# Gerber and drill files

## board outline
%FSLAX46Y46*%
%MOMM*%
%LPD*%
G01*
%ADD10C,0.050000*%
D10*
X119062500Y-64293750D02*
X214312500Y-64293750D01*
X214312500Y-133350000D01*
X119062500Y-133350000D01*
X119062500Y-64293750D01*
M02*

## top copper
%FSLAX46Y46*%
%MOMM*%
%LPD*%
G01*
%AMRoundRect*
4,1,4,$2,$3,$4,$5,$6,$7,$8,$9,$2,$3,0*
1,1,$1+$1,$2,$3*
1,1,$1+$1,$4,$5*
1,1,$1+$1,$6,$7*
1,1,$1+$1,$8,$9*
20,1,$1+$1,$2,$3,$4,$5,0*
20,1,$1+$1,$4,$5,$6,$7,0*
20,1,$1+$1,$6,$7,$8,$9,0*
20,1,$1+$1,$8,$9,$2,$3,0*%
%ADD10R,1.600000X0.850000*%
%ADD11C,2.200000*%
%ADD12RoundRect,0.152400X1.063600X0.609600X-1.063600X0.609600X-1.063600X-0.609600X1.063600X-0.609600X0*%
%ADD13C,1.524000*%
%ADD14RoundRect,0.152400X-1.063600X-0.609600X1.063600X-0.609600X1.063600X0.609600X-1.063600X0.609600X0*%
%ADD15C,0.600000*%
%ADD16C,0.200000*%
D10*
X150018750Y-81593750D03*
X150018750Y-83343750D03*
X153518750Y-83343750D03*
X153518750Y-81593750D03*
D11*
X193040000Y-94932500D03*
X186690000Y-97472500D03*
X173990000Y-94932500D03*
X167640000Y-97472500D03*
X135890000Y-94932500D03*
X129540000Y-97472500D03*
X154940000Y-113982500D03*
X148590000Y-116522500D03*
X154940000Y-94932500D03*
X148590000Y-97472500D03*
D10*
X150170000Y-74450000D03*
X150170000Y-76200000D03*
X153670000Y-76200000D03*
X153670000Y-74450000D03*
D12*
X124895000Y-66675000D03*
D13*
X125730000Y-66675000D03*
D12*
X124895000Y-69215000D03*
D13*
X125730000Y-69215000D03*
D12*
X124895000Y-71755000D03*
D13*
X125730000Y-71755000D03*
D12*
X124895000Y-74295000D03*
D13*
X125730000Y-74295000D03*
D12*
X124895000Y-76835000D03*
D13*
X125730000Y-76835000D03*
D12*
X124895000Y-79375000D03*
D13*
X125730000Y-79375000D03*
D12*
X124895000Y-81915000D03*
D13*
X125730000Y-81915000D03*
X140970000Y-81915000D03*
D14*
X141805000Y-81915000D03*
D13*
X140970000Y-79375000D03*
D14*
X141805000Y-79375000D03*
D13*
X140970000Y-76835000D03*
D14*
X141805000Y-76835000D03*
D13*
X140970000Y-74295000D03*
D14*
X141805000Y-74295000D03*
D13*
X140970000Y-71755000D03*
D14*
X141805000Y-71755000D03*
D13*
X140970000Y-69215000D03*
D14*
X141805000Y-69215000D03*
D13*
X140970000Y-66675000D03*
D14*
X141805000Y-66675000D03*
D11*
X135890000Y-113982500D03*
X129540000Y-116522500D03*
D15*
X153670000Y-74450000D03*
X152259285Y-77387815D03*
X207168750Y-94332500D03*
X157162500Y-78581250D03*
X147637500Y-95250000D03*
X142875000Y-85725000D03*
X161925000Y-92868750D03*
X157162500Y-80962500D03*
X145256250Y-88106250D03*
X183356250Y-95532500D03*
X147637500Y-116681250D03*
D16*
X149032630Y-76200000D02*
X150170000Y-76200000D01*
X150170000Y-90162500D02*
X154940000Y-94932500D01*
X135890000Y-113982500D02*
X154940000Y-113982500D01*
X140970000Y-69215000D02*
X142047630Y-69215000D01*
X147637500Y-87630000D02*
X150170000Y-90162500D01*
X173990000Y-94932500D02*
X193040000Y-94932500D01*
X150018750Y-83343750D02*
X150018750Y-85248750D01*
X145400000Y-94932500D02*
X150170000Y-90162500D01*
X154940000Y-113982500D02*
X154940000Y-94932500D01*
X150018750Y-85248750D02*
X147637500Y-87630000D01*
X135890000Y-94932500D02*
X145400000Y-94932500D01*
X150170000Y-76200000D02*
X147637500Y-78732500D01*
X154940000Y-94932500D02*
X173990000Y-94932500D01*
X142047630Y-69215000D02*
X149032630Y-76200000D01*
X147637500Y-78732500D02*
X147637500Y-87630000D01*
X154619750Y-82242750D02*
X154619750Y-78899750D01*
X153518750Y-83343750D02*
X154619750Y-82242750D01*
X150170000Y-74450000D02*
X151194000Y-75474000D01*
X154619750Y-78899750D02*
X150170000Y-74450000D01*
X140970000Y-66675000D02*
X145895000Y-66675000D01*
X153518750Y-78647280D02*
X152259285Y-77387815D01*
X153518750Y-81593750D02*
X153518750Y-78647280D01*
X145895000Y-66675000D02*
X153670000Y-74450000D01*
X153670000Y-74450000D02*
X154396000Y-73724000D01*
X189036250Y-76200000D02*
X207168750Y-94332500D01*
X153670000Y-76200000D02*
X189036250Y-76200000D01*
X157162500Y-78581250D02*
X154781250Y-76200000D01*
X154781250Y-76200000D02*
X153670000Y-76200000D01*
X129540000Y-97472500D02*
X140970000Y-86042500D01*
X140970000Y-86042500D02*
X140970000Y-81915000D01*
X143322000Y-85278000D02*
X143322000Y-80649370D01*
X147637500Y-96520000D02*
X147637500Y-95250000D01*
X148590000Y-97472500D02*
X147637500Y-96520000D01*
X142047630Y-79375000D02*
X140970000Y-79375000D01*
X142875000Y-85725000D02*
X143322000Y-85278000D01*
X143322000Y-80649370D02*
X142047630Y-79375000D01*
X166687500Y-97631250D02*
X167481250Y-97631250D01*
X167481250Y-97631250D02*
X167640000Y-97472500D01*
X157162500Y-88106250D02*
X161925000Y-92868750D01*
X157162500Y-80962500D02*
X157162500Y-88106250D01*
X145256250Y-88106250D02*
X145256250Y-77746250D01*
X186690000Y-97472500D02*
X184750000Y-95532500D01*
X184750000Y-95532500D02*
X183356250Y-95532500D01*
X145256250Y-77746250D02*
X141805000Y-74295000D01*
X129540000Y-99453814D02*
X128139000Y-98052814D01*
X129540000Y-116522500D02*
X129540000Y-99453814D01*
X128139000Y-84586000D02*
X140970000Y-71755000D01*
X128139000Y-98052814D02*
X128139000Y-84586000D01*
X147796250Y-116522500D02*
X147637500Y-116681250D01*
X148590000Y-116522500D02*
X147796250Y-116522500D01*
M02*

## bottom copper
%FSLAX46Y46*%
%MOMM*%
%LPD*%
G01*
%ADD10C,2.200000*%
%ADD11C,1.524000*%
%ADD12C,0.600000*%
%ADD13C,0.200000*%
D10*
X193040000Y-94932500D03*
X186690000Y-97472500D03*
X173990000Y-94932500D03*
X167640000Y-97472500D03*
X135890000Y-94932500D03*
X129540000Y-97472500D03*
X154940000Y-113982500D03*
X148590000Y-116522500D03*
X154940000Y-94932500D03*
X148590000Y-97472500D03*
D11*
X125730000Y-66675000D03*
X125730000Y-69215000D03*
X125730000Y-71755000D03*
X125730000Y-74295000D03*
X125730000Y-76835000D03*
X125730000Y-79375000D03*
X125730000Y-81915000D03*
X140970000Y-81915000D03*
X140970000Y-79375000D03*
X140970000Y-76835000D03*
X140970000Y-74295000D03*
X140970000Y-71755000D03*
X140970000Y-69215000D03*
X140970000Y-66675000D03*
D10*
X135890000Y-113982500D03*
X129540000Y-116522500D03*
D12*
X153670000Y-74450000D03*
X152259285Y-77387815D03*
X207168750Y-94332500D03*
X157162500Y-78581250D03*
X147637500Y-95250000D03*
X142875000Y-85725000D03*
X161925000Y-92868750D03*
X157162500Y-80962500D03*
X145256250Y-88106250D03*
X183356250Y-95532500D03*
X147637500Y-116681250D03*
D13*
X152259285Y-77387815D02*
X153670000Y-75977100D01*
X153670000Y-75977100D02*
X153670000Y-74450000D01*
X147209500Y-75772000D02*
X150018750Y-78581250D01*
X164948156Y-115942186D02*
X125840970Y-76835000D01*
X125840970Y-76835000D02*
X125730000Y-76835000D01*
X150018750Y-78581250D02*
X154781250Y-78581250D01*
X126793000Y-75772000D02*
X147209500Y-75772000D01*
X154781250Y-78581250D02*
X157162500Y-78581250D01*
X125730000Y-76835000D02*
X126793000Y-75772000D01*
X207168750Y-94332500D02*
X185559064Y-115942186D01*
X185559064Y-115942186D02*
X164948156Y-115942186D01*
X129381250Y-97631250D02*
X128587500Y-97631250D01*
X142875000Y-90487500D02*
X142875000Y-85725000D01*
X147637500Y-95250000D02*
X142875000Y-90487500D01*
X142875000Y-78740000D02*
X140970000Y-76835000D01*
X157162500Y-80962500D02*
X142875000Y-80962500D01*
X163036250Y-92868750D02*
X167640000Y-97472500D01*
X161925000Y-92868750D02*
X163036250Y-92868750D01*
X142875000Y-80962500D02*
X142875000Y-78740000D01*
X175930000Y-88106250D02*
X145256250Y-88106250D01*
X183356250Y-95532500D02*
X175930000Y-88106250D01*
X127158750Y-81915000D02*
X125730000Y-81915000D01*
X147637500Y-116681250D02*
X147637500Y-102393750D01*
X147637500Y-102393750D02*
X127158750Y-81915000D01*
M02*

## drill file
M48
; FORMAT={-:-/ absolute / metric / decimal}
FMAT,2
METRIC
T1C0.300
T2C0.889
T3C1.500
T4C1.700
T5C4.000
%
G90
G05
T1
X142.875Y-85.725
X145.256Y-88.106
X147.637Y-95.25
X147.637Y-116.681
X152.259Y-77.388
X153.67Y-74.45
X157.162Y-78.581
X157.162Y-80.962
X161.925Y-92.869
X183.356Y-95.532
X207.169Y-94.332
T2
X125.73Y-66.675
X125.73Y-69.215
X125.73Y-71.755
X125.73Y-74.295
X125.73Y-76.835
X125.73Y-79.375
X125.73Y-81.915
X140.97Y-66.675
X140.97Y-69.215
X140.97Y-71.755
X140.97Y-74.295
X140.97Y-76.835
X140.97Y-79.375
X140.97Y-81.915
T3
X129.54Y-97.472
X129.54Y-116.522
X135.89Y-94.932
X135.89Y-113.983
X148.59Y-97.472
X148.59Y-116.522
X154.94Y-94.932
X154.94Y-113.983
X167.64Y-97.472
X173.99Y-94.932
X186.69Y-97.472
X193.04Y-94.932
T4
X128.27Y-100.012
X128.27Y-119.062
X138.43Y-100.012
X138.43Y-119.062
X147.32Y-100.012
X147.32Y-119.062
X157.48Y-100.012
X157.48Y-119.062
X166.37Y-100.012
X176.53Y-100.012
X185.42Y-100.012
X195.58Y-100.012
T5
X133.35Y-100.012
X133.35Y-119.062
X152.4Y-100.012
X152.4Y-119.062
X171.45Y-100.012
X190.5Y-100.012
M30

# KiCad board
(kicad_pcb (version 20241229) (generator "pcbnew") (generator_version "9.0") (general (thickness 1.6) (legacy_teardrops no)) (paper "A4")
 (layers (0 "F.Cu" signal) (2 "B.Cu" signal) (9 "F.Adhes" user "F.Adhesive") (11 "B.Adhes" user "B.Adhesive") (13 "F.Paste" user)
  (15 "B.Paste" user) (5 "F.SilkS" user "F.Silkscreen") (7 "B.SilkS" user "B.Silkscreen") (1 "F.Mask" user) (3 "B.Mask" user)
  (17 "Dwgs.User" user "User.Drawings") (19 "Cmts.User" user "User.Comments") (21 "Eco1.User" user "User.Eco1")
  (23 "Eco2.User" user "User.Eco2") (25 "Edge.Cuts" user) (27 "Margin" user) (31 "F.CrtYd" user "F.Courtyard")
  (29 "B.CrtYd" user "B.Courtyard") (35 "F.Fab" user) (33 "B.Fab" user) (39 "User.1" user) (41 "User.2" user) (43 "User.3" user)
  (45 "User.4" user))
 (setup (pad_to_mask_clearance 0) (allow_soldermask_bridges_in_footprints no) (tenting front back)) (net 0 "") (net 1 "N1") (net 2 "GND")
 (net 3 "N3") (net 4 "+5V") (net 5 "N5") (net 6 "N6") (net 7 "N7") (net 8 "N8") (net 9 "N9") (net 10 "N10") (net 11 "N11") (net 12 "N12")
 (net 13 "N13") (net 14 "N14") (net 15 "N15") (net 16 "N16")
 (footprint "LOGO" (layer "F.Cu") (at 169.754101 70.000013)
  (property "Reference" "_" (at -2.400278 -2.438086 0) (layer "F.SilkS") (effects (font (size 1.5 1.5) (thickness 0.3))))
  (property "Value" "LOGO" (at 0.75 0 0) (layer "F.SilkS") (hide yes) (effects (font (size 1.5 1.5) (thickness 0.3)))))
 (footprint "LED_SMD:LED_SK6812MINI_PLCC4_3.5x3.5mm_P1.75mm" (layer "F.Cu") (at 151.76875 82.46875)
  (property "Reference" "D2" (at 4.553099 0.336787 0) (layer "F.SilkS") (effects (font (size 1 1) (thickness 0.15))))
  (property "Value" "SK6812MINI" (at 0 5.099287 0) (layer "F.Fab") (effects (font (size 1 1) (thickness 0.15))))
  (pad "1" smd rect (at -1.75 -0.875) (size 1.6 0.85) (layers "F.Cu" "F.Mask" "F.Paste") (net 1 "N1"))
  (pad "2" smd rect (at -1.75 0.875) (size 1.6 0.85) (layers "F.Cu" "F.Mask" "F.Paste") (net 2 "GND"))
  (pad "3" smd rect (at 1.75 0.875) (size 1.6 0.85) (layers "F.Cu" "F.Mask" "F.Paste") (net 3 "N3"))
  (pad "4" smd rect (at 1.75 -0.875) (size 1.6 0.85) (layers "F.Cu" "F.Mask" "F.Paste") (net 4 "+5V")))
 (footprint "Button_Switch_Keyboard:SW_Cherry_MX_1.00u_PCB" (layer "F.Cu") (at 193.04 94.9325)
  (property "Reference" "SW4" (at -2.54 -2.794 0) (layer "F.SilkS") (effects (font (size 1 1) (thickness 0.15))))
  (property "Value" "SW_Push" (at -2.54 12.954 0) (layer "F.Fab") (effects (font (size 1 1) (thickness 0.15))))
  (pad "" np_thru_hole circle (at -7.62 5.08) (size 1.7 1.7) (drill 1.7) (layers "*.Cu" "*.Mask"))
  (pad "" np_thru_hole circle (at -2.54 5.08) (size 4 4) (drill 4) (layers "*.Cu" "*.Mask"))
  (pad "" np_thru_hole circle (at 2.54 5.08) (size 1.7 1.7) (drill 1.7) (layers "*.Cu" "*.Mask"))
  (pad "1" thru_hole circle (at 0 0) (size 2.2 2.2) (drill 1.5) (layers "*.Cu" "*.Mask") (remove_unused_layers no) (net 2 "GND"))
  (pad "2" thru_hole circle (at -6.35 2.54) (size 2.2 2.2) (drill 1.5) (layers "*.Cu" "*.Mask") (remove_unused_layers no) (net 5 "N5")))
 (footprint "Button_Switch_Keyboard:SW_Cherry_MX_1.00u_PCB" (layer "F.Cu") (at 173.99 94.9325)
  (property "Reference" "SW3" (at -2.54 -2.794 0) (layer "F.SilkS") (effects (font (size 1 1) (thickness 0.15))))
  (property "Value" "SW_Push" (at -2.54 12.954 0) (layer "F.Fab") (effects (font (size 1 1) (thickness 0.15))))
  (pad "" np_thru_hole circle (at -7.62 5.08) (size 1.7 1.7) (drill 1.7) (layers "*.Cu" "*.Mask"))
  (pad "" np_thru_hole circle (at -2.54 5.08) (size 4 4) (drill 4) (layers "*.Cu" "*.Mask"))
  (pad "" np_thru_hole circle (at 2.54 5.08) (size 1.7 1.7) (drill 1.7) (layers "*.Cu" "*.Mask"))
  (pad "1" thru_hole circle (at 0 0) (size 2.2 2.2) (drill 1.5) (layers "*.Cu" "*.Mask") (remove_unused_layers no) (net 2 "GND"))
  (pad "2" thru_hole circle (at -6.35 2.54) (size 2.2 2.2) (drill 1.5) (layers "*.Cu" "*.Mask") (remove_unused_layers no) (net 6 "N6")))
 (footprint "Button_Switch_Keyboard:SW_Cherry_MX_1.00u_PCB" (layer "F.Cu") (at 135.89 94.9325)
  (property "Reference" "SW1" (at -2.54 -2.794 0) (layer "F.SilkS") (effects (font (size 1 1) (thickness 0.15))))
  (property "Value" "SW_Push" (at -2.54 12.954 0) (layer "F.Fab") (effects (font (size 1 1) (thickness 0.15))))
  (pad "" np_thru_hole circle (at -7.62 5.08) (size 1.7 1.7) (drill 1.7) (layers "*.Cu" "*.Mask"))
  (pad "" np_thru_hole circle (at -2.54 5.08) (size 4 4) (drill 4) (layers "*.Cu" "*.Mask"))
  (pad "" np_thru_hole circle (at 2.54 5.08) (size 1.7 1.7) (drill 1.7) (layers "*.Cu" "*.Mask"))
  (pad "1" thru_hole circle (at 0 0) (size 2.2 2.2) (drill 1.5) (layers "*.Cu" "*.Mask") (remove_unused_layers no) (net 2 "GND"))
  (pad "2" thru_hole circle (at -6.35 2.54) (size 2.2 2.2) (drill 1.5) (layers "*.Cu" "*.Mask") (remove_unused_layers no) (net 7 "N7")))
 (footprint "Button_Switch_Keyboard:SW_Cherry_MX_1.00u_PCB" (layer "F.Cu") (at 154.94 113.9825)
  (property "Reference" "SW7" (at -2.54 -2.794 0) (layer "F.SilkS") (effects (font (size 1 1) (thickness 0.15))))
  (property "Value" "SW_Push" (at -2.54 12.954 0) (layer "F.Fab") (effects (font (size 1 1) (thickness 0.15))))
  (pad "" np_thru_hole circle (at -7.62 5.08) (size 1.7 1.7) (drill 1.7) (layers "*.Cu" "*.Mask"))
  (pad "" np_thru_hole circle (at -2.54 5.08) (size 4 4) (drill 4) (layers "*.Cu" "*.Mask"))
  (pad "" np_thru_hole circle (at 2.54 5.08) (size 1.7 1.7) (drill 1.7) (layers "*.Cu" "*.Mask"))
  (pad "1" thru_hole circle (at 0 0) (size 2.2 2.2) (drill 1.5) (layers "*.Cu" "*.Mask") (remove_unused_layers no) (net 2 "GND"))
  (pad "2" thru_hole circle (at -6.35 2.54) (size 2.2 2.2) (drill 1.5) (layers "*.Cu" "*.Mask") (remove_unused_layers no) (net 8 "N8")))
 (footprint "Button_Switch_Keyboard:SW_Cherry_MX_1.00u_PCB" (layer "F.Cu") (at 154.94 94.9325)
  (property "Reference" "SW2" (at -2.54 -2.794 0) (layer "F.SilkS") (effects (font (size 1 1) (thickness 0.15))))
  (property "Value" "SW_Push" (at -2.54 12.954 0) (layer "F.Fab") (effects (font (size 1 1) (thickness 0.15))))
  (pad "" np_thru_hole circle (at -7.62 5.08) (size 1.7 1.7) (drill 1.7) (layers "*.Cu" "*.Mask"))
  (pad "" np_thru_hole circle (at -2.54 5.08) (size 4 4) (drill 4) (layers "*.Cu" "*.Mask"))
  (pad "" np_thru_hole circle (at 2.54 5.08) (size 1.7 1.7) (drill 1.7) (layers "*.Cu" "*.Mask"))
  (pad "1" thru_hole circle (at 0 0) (size 2.2 2.2) (drill 1.5) (layers "*.Cu" "*.Mask") (remove_unused_layers no) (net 2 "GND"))
  (pad "2" thru_hole circle (at -6.35 2.54) (size 2.2 2.2) (drill 1.5) (layers "*.Cu" "*.Mask") (remove_unused_layers no) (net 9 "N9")))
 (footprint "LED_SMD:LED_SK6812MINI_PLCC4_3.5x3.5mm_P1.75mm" (layer "F.Cu") (at 151.92 75.325)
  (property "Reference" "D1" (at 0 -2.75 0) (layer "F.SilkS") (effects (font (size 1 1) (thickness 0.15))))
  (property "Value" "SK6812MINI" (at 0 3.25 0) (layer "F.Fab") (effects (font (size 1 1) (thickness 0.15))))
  (pad "1" smd rect (at -1.75 -0.875) (size 1.6 0.85) (layers "F.Cu" "F.Mask" "F.Paste") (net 3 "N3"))
  (pad "2" smd rect (at -1.75 0.875) (size 1.6 0.85) (layers "F.Cu" "F.Mask" "F.Paste") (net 2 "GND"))
  (pad "3" smd rect (at 1.75 0.875) (size 1.6 0.85) (layers "F.Cu" "F.Mask" "F.Paste") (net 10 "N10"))
  (pad "4" smd rect (at 1.75 -0.875) (size 1.6 0.85) (layers "F.Cu" "F.Mask" "F.Paste") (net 4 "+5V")))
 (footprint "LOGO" (layer "F.Cu") (at 196.914142 78.488281)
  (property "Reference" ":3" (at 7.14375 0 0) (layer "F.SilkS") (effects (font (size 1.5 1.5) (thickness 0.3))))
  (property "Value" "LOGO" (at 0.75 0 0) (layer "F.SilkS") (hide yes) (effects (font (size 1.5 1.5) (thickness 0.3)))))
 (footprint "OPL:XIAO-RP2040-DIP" (layer "F.Cu") (at 133.35 74.295)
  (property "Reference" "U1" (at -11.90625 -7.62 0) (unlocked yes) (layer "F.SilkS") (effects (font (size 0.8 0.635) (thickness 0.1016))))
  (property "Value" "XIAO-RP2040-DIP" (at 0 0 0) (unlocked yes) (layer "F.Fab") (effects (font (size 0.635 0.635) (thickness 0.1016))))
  (pad "1" smd roundrect (at -8.455 -7.62 180) (size 2.432 1.524) (layers "F.Cu" "F.Mask") (roundrect_rratio 0.1) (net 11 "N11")
   (thermal_bridge_angle 45))
  (pad "1" thru_hole circle (at -7.62 -7.62 180) (size 1.524 1.524) (drill 0.889) (layers "*.Cu" "*.Mask") (remove_unused_layers no)
   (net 11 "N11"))
  (pad "2" smd roundrect (at -8.455 -5.08 180) (size 2.432 1.524) (layers "F.Cu" "F.Mask") (roundrect_rratio 0.1) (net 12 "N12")
   (thermal_bridge_angle 45))
  (pad "2" thru_hole circle (at -7.62 -5.08 180) (size 1.524 1.524) (drill 0.889) (layers "*.Cu" "*.Mask") (remove_unused_layers no)
   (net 12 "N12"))
  (pad "3" smd roundrect (at -8.455 -2.54 180) (size 2.432 1.524) (layers "F.Cu" "F.Mask") (roundrect_rratio 0.1) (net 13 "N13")
   (thermal_bridge_angle 45))
  (pad "3" thru_hole circle (at -7.62 -2.54 180) (size 1.524 1.524) (drill 0.889) (layers "*.Cu" "*.Mask") (remove_unused_layers no)
   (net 13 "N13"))
  (pad "4" smd roundrect (at -8.455 0 180) (size 2.432 1.524) (layers "F.Cu" "F.Mask") (roundrect_rratio 0.1) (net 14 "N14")
   (thermal_bridge_angle 45))
  (pad "4" thru_hole circle (at -7.62 0 180) (size 1.524 1.524) (drill 0.889) (layers "*.Cu" "*.Mask") (remove_unused_layers no)
   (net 14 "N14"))
  (pad "5" smd roundrect (at -8.455 2.54 180) (size 2.432 1.524) (layers "F.Cu" "F.Mask") (roundrect_rratio 0.1) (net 10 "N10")
   (thermal_bridge_angle 45))
  (pad "5" thru_hole circle (at -7.62 2.54 180) (size 1.524 1.524) (drill 0.889) (layers "*.Cu" "*.Mask") (remove_unused_layers no)
   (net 10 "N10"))
  (pad "6" smd roundrect (at -8.455 5.08 180) (size 2.432 1.524) (layers "F.Cu" "F.Mask") (roundrect_rratio 0.1) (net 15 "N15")
   (thermal_bridge_angle 45))
  (pad "6" thru_hole circle (at -7.62 5.08 180) (size 1.524 1.524) (drill 0.889) (layers "*.Cu" "*.Mask") (remove_unused_layers no)
   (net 15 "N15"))
  (pad "7" smd roundrect (at -8.455 7.62 180) (size 2.432 1.524) (layers "F.Cu" "F.Mask") (roundrect_rratio 0.1) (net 8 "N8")
   (thermal_bridge_angle 45))
  (pad "7" thru_hole circle (at -7.62 7.62 180) (size 1.524 1.524) (drill 0.889) (layers "*.Cu" "*.Mask") (remove_unused_layers no)
   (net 8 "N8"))
  (pad "8" thru_hole circle (at 7.62 7.62) (size 1.524 1.524) (drill 0.889) (layers "*.Cu" "*.Mask") (remove_unused_layers no) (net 7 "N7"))
  (pad "8" smd roundrect (at 8.455 7.62) (size 2.432 1.524) (layers "F.Cu" "F.Mask") (roundrect_rratio 0.1) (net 7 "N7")
   (thermal_bridge_angle 45))
  (pad "9" thru_hole circle (at 7.62 5.08) (size 1.524 1.524) (drill 0.889) (layers "*.Cu" "*.Mask") (remove_unused_layers no) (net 9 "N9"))
  (pad "9" smd roundrect (at 8.455 5.08) (size 2.432 1.524) (layers "F.Cu" "F.Mask") (roundrect_rratio 0.1) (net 9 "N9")
   (thermal_bridge_angle 45))
  (pad "10" thru_hole circle (at 7.62 2.54) (size 1.524 1.524) (drill 0.889) (layers "*.Cu" "*.Mask") (remove_unused_layers no) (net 6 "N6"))
  (pad "10" smd roundrect (at 8.455 2.54) (size 2.432 1.524) (layers "F.Cu" "F.Mask") (roundrect_rratio 0.1) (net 6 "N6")
   (thermal_bridge_angle 45))
  (pad "11" thru_hole circle (at 7.62 0) (size 1.524 1.524) (drill 0.889) (layers "*.Cu" "*.Mask") (remove_unused_layers no) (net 5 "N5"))
  (pad "11" smd roundrect (at 8.455 0) (size 2.432 1.524) (layers "F.Cu" "F.Mask") (roundrect_rratio 0.1) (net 5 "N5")
   (thermal_bridge_angle 45))
  (pad "12" thru_hole circle (at 7.62 -2.54) (size 1.524 1.524) (drill 0.889) (layers "*.Cu" "*.Mask") (remove_unused_layers no)
   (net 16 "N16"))
  (pad "12" smd roundrect (at 8.455 -2.54) (size 2.432 1.524) (layers "F.Cu" "F.Mask") (roundrect_rratio 0.1) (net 16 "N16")
   (thermal_bridge_angle 45))
  (pad "13" thru_hole circle (at 7.62 -5.08) (size 1.524 1.524) (drill 0.889) (layers "*.Cu" "*.Mask") (remove_unused_layers no)
   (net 2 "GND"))
  (pad "13" smd roundrect (at 8.455 -5.08) (size 2.432 1.524) (layers "F.Cu" "F.Mask") (roundrect_rratio 0.1) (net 2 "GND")
   (thermal_bridge_angle 45))
  (pad "14" thru_hole circle (at 7.62 -7.62) (size 1.524 1.524) (drill 0.889) (layers "*.Cu" "*.Mask") (remove_unused_layers no)
   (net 4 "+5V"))
  (pad "14" smd roundrect (at 8.455 -7.62) (size 2.432 1.524) (layers "F.Cu" "F.Mask") (roundrect_rratio 0.1) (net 4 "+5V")
   (thermal_bridge_angle 45)))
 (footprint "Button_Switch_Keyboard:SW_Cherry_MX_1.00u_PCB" (layer "F.Cu") (at 135.89 113.9825)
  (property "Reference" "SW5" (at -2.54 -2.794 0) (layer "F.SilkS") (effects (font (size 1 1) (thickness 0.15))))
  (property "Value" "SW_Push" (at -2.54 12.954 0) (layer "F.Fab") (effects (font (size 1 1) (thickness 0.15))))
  (pad "" np_thru_hole circle (at -7.62 5.08) (size 1.7 1.7) (drill 1.7) (layers "*.Cu" "*.Mask"))
  (pad "" np_thru_hole circle (at -2.54 5.08) (size 4 4) (drill 4) (layers "*.Cu" "*.Mask"))
  (pad "" np_thru_hole circle (at 2.54 5.08) (size 1.7 1.7) (drill 1.7) (layers "*.Cu" "*.Mask"))
  (pad "1" thru_hole circle (at 0 0) (size 2.2 2.2) (drill 1.5) (layers "*.Cu" "*.Mask") (remove_unused_layers no) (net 2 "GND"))
  (pad "2" thru_hole circle (at -6.35 2.54) (size 2.2 2.2) (drill 1.5) (layers "*.Cu" "*.Mask") (remove_unused_layers no) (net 16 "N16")))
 (gr_rect (start 119.0625 64.29375) (end 214.3125 133.35) (stroke (width 0.05) (type default)) (fill no) (layer "Edge.Cuts"))
 (segment (start 149.03263 76.2) (end 150.17 76.2) (width 0.2) (layer "F.Cu") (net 2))
 (segment (start 150.17 90.1625) (end 154.94 94.9325) (width 0.2) (layer "F.Cu") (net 2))
 (segment (start 135.89 113.9825) (end 154.94 113.9825) (width 0.2) (layer "F.Cu") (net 2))
 (segment (start 140.97 69.215) (end 142.04763 69.215) (width 0.2) (layer "F.Cu") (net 2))
 (segment (start 147.6375 87.63) (end 150.17 90.1625) (width 0.2) (layer "F.Cu") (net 2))
 (segment (start 173.99 94.9325) (end 193.04 94.9325) (width 0.2) (layer "F.Cu") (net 2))
 (segment (start 150.01875 83.34375) (end 150.01875 85.24875) (width 0.2) (layer "F.Cu") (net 2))
 (segment (start 145.4 94.9325) (end 150.17 90.1625) (width 0.2) (layer "F.Cu") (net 2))
 (segment (start 154.94 113.9825) (end 154.94 94.9325) (width 0.2) (layer "F.Cu") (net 2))
 (segment (start 150.01875 85.24875) (end 147.6375 87.63) (width 0.2) (layer "F.Cu") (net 2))
 (segment (start 135.89 94.9325) (end 145.4 94.9325) (width 0.2) (layer "F.Cu") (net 2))
 (segment (start 150.17 76.2) (end 147.6375 78.7325) (width 0.2) (layer "F.Cu") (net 2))
 (segment (start 154.94 94.9325) (end 173.99 94.9325) (width 0.2) (layer "F.Cu") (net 2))
 (segment (start 142.04763 69.215) (end 149.03263 76.2) (width 0.2) (layer "F.Cu") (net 2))
 (segment (start 147.6375 78.7325) (end 147.6375 87.63) (width 0.2) (layer "F.Cu") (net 2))
 (segment (start 154.61975 82.24275) (end 154.61975 78.89975) (width 0.2) (layer "F.Cu") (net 3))
 (segment (start 153.51875 83.34375) (end 154.61975 82.24275) (width 0.2) (layer "F.Cu") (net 3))
 (segment (start 150.17 74.45) (end 151.194 75.474) (width 0.2) (layer "F.Cu") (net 3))
 (segment (start 154.61975 78.89975) (end 150.17 74.45) (width 0.2) (layer "F.Cu") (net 3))
 (segment (start 140.97 66.675) (end 145.895 66.675) (width 0.2) (layer "F.Cu") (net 4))
 (segment (start 153.51875 78.64728) (end 152.259285 77.387815) (width 0.2) (layer "F.Cu") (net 4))
 (segment (start 153.51875 81.59375) (end 153.51875 78.64728) (width 0.2) (layer "F.Cu") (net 4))
 (segment (start 145.895 66.675) (end 153.67 74.45) (width 0.2) (layer "F.Cu") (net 4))
 (segment (start 153.67 74.45) (end 154.396 73.724) (width 0.2) (layer "F.Cu") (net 4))
 (via (at 153.67 74.45) (size 0.6) (drill 0.3) (layers "F.Cu" "B.Cu") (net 4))
 (via (at 152.259285 77.387815) (size 0.6) (drill 0.3) (layers "F.Cu" "B.Cu") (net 4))
 (segment (start 152.259285 77.387815) (end 153.67 75.9771) (width 0.2) (layer "B.Cu") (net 4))
 (segment (start 153.67 75.9771) (end 153.67 74.45) (width 0.2) (layer "B.Cu") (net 4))
 (segment (start 189.03625 76.2) (end 207.16875 94.3325) (width 0.2) (layer "F.Cu") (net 10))
 (segment (start 153.67 76.2) (end 189.03625 76.2) (width 0.2) (layer "F.Cu") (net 10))
 (segment (start 157.1625 78.58125) (end 154.78125 76.2) (width 0.2) (layer "F.Cu") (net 10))
 (segment (start 154.78125 76.2) (end 153.67 76.2) (width 0.2) (layer "F.Cu") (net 10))
 (via (at 207.16875 94.3325) (size 0.6) (drill 0.3) (layers "F.Cu" "B.Cu") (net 10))
 (via (at 157.1625 78.58125) (size 0.6) (drill 0.3) (layers "F.Cu" "B.Cu") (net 10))
 (segment (start 147.2095 75.772) (end 150.01875 78.58125) (width 0.2) (layer "B.Cu") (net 10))
 (segment (start 164.948156 115.942186) (end 125.84097 76.835) (width 0.2) (layer "B.Cu") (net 10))
 (segment (start 125.84097 76.835) (end 125.73 76.835) (width 0.2) (layer "B.Cu") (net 10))
 (segment (start 150.01875 78.58125) (end 154.78125 78.58125) (width 0.2) (layer "B.Cu") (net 10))
 (segment (start 126.793 75.772) (end 147.2095 75.772) (width 0.2) (layer "B.Cu") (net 10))
 (segment (start 154.78125 78.58125) (end 157.1625 78.58125) (width 0.2) (layer "B.Cu") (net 10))
 (segment (start 125.73 76.835) (end 126.793 75.772) (width 0.2) (layer "B.Cu") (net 10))
 (segment (start 207.16875 94.3325) (end 185.559064 115.942186) (width 0.2) (layer "B.Cu") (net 10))
 (segment (start 185.559064 115.942186) (end 164.948156 115.942186) (width 0.2) (layer "B.Cu") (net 10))
 (segment (start 129.54 97.4725) (end 140.97 86.0425) (width 0.2) (layer "F.Cu") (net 7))
 (segment (start 140.97 86.0425) (end 140.97 81.915) (width 0.2) (layer "F.Cu") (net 7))
 (segment (start 129.38125 97.63125) (end 128.5875 97.63125) (width 0.2) (layer "B.Cu") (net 7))
 (segment (start 143.322 85.278) (end 143.322 80.64937) (width 0.2) (layer "F.Cu") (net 9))
 (segment (start 147.6375 96.52) (end 147.6375 95.25) (width 0.2) (layer "F.Cu") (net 9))
 (segment (start 148.59 97.4725) (end 147.6375 96.52) (width 0.2) (layer "F.Cu") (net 9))
 (segment (start 142.04763 79.375) (end 140.97 79.375) (width 0.2) (layer "F.Cu") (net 9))
 (segment (start 142.875 85.725) (end 143.322 85.278) (width 0.2) (layer "F.Cu") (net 9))
 (segment (start 143.322 80.64937) (end 142.04763 79.375) (width 0.2) (layer "F.Cu") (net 9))
 (via (at 147.6375 95.25) (size 0.6) (drill 0.3) (layers "F.Cu" "B.Cu") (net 9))
 (via (at 142.875 85.725) (size 0.6) (drill 0.3) (layers "F.Cu" "B.Cu") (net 9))
 (segment (start 142.875 90.4875) (end 142.875 85.725) (width 0.2) (layer "B.Cu") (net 9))
 (segment (start 147.6375 95.25) (end 142.875 90.4875) (width 0.2) (layer "B.Cu") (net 9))
 (segment (start 166.6875 97.63125) (end 167.48125 97.63125) (width 0.2) (layer "F.Cu") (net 6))
 (segment (start 167.48125 97.63125) (end 167.64 97.4725) (width 0.2) (layer "F.Cu") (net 6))
 (segment (start 157.1625 88.10625) (end 161.925 92.86875) (width 0.2) (layer "F.Cu") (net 6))
 (segment (start 157.1625 80.9625) (end 157.1625 88.10625) (width 0.2) (layer "F.Cu") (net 6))
 (via (at 161.925 92.86875) (size 0.6) (drill 0.3) (layers "F.Cu" "B.Cu") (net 6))
 (via (at 157.1625 80.9625) (size 0.6) (drill 0.3) (layers "F.Cu" "B.Cu") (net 6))
 (segment (start 142.875 78.74) (end 140.97 76.835) (width 0.2) (layer "B.Cu") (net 6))
 (segment (start 157.1625 80.9625) (end 142.875 80.9625) (width 0.2) (layer "B.Cu") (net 6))
 (segment (start 163.03625 92.86875) (end 167.64 97.4725) (width 0.2) (layer "B.Cu") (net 6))
 (segment (start 161.925 92.86875) (end 163.03625 92.86875) (width 0.2) (layer "B.Cu") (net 6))
 (segment (start 142.875 80.9625) (end 142.875 78.74) (width 0.2) (layer "B.Cu") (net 6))
 (segment (start 145.25625 88.10625) (end 145.25625 77.74625) (width 0.2) (layer "F.Cu") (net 5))
 (segment (start 186.69 97.4725) (end 184.75 95.5325) (width 0.2) (layer "F.Cu") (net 5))
 (segment (start 184.75 95.5325) (end 183.35625 95.5325) (width 0.2) (layer "F.Cu") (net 5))
 (segment (start 145.25625 77.74625) (end 141.805 74.295) (width 0.2) (layer "F.Cu") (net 5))
 (via (at 145.25625 88.10625) (size 0.6) (drill 0.3) (layers "F.Cu" "B.Cu") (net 5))
 (via (at 183.35625 95.5325) (size 0.6) (drill 0.3) (layers "F.Cu" "B.Cu") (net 5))
 (segment (start 175.93 88.10625) (end 145.25625 88.10625) (width 0.2) (layer "B.Cu") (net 5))
 (segment (start 183.35625 95.5325) (end 175.93 88.10625) (width 0.2) (layer "B.Cu") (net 5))
 (segment (start 129.54 99.453814) (end 128.139 98.052814) (width 0.2) (layer "F.Cu") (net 16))
 (segment (start 129.54 116.5225) (end 129.54 99.453814) (width 0.2) (layer "F.Cu") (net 16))
 (segment (start 128.139 84.586) (end 140.97 71.755) (width 0.2) (layer "F.Cu") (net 16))
 (segment (start 128.139 98.052814) (end 128.139 84.586) (width 0.2) (layer "F.Cu") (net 16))
 (segment (start 147.79625 116.5225) (end 147.6375 116.68125) (width 0.2) (layer "F.Cu") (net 8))
 (segment (start 148.59 116.5225) (end 147.79625 116.5225) (width 0.2) (layer "F.Cu") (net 8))
 (via (at 147.6375 116.68125) (size 0.6) (drill 0.3) (layers "F.Cu" "B.Cu") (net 8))
 (segment (start 127.15875 81.915) (end 125.73 81.915) (width 0.2) (layer "B.Cu") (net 8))
 (segment (start 147.6375 116.68125) (end 147.6375 102.39375) (width 0.2) (layer "B.Cu") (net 8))
 (segment (start 147.6375 102.39375) (end 127.15875 81.915) (width 0.2) (layer "B.Cu") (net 8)))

